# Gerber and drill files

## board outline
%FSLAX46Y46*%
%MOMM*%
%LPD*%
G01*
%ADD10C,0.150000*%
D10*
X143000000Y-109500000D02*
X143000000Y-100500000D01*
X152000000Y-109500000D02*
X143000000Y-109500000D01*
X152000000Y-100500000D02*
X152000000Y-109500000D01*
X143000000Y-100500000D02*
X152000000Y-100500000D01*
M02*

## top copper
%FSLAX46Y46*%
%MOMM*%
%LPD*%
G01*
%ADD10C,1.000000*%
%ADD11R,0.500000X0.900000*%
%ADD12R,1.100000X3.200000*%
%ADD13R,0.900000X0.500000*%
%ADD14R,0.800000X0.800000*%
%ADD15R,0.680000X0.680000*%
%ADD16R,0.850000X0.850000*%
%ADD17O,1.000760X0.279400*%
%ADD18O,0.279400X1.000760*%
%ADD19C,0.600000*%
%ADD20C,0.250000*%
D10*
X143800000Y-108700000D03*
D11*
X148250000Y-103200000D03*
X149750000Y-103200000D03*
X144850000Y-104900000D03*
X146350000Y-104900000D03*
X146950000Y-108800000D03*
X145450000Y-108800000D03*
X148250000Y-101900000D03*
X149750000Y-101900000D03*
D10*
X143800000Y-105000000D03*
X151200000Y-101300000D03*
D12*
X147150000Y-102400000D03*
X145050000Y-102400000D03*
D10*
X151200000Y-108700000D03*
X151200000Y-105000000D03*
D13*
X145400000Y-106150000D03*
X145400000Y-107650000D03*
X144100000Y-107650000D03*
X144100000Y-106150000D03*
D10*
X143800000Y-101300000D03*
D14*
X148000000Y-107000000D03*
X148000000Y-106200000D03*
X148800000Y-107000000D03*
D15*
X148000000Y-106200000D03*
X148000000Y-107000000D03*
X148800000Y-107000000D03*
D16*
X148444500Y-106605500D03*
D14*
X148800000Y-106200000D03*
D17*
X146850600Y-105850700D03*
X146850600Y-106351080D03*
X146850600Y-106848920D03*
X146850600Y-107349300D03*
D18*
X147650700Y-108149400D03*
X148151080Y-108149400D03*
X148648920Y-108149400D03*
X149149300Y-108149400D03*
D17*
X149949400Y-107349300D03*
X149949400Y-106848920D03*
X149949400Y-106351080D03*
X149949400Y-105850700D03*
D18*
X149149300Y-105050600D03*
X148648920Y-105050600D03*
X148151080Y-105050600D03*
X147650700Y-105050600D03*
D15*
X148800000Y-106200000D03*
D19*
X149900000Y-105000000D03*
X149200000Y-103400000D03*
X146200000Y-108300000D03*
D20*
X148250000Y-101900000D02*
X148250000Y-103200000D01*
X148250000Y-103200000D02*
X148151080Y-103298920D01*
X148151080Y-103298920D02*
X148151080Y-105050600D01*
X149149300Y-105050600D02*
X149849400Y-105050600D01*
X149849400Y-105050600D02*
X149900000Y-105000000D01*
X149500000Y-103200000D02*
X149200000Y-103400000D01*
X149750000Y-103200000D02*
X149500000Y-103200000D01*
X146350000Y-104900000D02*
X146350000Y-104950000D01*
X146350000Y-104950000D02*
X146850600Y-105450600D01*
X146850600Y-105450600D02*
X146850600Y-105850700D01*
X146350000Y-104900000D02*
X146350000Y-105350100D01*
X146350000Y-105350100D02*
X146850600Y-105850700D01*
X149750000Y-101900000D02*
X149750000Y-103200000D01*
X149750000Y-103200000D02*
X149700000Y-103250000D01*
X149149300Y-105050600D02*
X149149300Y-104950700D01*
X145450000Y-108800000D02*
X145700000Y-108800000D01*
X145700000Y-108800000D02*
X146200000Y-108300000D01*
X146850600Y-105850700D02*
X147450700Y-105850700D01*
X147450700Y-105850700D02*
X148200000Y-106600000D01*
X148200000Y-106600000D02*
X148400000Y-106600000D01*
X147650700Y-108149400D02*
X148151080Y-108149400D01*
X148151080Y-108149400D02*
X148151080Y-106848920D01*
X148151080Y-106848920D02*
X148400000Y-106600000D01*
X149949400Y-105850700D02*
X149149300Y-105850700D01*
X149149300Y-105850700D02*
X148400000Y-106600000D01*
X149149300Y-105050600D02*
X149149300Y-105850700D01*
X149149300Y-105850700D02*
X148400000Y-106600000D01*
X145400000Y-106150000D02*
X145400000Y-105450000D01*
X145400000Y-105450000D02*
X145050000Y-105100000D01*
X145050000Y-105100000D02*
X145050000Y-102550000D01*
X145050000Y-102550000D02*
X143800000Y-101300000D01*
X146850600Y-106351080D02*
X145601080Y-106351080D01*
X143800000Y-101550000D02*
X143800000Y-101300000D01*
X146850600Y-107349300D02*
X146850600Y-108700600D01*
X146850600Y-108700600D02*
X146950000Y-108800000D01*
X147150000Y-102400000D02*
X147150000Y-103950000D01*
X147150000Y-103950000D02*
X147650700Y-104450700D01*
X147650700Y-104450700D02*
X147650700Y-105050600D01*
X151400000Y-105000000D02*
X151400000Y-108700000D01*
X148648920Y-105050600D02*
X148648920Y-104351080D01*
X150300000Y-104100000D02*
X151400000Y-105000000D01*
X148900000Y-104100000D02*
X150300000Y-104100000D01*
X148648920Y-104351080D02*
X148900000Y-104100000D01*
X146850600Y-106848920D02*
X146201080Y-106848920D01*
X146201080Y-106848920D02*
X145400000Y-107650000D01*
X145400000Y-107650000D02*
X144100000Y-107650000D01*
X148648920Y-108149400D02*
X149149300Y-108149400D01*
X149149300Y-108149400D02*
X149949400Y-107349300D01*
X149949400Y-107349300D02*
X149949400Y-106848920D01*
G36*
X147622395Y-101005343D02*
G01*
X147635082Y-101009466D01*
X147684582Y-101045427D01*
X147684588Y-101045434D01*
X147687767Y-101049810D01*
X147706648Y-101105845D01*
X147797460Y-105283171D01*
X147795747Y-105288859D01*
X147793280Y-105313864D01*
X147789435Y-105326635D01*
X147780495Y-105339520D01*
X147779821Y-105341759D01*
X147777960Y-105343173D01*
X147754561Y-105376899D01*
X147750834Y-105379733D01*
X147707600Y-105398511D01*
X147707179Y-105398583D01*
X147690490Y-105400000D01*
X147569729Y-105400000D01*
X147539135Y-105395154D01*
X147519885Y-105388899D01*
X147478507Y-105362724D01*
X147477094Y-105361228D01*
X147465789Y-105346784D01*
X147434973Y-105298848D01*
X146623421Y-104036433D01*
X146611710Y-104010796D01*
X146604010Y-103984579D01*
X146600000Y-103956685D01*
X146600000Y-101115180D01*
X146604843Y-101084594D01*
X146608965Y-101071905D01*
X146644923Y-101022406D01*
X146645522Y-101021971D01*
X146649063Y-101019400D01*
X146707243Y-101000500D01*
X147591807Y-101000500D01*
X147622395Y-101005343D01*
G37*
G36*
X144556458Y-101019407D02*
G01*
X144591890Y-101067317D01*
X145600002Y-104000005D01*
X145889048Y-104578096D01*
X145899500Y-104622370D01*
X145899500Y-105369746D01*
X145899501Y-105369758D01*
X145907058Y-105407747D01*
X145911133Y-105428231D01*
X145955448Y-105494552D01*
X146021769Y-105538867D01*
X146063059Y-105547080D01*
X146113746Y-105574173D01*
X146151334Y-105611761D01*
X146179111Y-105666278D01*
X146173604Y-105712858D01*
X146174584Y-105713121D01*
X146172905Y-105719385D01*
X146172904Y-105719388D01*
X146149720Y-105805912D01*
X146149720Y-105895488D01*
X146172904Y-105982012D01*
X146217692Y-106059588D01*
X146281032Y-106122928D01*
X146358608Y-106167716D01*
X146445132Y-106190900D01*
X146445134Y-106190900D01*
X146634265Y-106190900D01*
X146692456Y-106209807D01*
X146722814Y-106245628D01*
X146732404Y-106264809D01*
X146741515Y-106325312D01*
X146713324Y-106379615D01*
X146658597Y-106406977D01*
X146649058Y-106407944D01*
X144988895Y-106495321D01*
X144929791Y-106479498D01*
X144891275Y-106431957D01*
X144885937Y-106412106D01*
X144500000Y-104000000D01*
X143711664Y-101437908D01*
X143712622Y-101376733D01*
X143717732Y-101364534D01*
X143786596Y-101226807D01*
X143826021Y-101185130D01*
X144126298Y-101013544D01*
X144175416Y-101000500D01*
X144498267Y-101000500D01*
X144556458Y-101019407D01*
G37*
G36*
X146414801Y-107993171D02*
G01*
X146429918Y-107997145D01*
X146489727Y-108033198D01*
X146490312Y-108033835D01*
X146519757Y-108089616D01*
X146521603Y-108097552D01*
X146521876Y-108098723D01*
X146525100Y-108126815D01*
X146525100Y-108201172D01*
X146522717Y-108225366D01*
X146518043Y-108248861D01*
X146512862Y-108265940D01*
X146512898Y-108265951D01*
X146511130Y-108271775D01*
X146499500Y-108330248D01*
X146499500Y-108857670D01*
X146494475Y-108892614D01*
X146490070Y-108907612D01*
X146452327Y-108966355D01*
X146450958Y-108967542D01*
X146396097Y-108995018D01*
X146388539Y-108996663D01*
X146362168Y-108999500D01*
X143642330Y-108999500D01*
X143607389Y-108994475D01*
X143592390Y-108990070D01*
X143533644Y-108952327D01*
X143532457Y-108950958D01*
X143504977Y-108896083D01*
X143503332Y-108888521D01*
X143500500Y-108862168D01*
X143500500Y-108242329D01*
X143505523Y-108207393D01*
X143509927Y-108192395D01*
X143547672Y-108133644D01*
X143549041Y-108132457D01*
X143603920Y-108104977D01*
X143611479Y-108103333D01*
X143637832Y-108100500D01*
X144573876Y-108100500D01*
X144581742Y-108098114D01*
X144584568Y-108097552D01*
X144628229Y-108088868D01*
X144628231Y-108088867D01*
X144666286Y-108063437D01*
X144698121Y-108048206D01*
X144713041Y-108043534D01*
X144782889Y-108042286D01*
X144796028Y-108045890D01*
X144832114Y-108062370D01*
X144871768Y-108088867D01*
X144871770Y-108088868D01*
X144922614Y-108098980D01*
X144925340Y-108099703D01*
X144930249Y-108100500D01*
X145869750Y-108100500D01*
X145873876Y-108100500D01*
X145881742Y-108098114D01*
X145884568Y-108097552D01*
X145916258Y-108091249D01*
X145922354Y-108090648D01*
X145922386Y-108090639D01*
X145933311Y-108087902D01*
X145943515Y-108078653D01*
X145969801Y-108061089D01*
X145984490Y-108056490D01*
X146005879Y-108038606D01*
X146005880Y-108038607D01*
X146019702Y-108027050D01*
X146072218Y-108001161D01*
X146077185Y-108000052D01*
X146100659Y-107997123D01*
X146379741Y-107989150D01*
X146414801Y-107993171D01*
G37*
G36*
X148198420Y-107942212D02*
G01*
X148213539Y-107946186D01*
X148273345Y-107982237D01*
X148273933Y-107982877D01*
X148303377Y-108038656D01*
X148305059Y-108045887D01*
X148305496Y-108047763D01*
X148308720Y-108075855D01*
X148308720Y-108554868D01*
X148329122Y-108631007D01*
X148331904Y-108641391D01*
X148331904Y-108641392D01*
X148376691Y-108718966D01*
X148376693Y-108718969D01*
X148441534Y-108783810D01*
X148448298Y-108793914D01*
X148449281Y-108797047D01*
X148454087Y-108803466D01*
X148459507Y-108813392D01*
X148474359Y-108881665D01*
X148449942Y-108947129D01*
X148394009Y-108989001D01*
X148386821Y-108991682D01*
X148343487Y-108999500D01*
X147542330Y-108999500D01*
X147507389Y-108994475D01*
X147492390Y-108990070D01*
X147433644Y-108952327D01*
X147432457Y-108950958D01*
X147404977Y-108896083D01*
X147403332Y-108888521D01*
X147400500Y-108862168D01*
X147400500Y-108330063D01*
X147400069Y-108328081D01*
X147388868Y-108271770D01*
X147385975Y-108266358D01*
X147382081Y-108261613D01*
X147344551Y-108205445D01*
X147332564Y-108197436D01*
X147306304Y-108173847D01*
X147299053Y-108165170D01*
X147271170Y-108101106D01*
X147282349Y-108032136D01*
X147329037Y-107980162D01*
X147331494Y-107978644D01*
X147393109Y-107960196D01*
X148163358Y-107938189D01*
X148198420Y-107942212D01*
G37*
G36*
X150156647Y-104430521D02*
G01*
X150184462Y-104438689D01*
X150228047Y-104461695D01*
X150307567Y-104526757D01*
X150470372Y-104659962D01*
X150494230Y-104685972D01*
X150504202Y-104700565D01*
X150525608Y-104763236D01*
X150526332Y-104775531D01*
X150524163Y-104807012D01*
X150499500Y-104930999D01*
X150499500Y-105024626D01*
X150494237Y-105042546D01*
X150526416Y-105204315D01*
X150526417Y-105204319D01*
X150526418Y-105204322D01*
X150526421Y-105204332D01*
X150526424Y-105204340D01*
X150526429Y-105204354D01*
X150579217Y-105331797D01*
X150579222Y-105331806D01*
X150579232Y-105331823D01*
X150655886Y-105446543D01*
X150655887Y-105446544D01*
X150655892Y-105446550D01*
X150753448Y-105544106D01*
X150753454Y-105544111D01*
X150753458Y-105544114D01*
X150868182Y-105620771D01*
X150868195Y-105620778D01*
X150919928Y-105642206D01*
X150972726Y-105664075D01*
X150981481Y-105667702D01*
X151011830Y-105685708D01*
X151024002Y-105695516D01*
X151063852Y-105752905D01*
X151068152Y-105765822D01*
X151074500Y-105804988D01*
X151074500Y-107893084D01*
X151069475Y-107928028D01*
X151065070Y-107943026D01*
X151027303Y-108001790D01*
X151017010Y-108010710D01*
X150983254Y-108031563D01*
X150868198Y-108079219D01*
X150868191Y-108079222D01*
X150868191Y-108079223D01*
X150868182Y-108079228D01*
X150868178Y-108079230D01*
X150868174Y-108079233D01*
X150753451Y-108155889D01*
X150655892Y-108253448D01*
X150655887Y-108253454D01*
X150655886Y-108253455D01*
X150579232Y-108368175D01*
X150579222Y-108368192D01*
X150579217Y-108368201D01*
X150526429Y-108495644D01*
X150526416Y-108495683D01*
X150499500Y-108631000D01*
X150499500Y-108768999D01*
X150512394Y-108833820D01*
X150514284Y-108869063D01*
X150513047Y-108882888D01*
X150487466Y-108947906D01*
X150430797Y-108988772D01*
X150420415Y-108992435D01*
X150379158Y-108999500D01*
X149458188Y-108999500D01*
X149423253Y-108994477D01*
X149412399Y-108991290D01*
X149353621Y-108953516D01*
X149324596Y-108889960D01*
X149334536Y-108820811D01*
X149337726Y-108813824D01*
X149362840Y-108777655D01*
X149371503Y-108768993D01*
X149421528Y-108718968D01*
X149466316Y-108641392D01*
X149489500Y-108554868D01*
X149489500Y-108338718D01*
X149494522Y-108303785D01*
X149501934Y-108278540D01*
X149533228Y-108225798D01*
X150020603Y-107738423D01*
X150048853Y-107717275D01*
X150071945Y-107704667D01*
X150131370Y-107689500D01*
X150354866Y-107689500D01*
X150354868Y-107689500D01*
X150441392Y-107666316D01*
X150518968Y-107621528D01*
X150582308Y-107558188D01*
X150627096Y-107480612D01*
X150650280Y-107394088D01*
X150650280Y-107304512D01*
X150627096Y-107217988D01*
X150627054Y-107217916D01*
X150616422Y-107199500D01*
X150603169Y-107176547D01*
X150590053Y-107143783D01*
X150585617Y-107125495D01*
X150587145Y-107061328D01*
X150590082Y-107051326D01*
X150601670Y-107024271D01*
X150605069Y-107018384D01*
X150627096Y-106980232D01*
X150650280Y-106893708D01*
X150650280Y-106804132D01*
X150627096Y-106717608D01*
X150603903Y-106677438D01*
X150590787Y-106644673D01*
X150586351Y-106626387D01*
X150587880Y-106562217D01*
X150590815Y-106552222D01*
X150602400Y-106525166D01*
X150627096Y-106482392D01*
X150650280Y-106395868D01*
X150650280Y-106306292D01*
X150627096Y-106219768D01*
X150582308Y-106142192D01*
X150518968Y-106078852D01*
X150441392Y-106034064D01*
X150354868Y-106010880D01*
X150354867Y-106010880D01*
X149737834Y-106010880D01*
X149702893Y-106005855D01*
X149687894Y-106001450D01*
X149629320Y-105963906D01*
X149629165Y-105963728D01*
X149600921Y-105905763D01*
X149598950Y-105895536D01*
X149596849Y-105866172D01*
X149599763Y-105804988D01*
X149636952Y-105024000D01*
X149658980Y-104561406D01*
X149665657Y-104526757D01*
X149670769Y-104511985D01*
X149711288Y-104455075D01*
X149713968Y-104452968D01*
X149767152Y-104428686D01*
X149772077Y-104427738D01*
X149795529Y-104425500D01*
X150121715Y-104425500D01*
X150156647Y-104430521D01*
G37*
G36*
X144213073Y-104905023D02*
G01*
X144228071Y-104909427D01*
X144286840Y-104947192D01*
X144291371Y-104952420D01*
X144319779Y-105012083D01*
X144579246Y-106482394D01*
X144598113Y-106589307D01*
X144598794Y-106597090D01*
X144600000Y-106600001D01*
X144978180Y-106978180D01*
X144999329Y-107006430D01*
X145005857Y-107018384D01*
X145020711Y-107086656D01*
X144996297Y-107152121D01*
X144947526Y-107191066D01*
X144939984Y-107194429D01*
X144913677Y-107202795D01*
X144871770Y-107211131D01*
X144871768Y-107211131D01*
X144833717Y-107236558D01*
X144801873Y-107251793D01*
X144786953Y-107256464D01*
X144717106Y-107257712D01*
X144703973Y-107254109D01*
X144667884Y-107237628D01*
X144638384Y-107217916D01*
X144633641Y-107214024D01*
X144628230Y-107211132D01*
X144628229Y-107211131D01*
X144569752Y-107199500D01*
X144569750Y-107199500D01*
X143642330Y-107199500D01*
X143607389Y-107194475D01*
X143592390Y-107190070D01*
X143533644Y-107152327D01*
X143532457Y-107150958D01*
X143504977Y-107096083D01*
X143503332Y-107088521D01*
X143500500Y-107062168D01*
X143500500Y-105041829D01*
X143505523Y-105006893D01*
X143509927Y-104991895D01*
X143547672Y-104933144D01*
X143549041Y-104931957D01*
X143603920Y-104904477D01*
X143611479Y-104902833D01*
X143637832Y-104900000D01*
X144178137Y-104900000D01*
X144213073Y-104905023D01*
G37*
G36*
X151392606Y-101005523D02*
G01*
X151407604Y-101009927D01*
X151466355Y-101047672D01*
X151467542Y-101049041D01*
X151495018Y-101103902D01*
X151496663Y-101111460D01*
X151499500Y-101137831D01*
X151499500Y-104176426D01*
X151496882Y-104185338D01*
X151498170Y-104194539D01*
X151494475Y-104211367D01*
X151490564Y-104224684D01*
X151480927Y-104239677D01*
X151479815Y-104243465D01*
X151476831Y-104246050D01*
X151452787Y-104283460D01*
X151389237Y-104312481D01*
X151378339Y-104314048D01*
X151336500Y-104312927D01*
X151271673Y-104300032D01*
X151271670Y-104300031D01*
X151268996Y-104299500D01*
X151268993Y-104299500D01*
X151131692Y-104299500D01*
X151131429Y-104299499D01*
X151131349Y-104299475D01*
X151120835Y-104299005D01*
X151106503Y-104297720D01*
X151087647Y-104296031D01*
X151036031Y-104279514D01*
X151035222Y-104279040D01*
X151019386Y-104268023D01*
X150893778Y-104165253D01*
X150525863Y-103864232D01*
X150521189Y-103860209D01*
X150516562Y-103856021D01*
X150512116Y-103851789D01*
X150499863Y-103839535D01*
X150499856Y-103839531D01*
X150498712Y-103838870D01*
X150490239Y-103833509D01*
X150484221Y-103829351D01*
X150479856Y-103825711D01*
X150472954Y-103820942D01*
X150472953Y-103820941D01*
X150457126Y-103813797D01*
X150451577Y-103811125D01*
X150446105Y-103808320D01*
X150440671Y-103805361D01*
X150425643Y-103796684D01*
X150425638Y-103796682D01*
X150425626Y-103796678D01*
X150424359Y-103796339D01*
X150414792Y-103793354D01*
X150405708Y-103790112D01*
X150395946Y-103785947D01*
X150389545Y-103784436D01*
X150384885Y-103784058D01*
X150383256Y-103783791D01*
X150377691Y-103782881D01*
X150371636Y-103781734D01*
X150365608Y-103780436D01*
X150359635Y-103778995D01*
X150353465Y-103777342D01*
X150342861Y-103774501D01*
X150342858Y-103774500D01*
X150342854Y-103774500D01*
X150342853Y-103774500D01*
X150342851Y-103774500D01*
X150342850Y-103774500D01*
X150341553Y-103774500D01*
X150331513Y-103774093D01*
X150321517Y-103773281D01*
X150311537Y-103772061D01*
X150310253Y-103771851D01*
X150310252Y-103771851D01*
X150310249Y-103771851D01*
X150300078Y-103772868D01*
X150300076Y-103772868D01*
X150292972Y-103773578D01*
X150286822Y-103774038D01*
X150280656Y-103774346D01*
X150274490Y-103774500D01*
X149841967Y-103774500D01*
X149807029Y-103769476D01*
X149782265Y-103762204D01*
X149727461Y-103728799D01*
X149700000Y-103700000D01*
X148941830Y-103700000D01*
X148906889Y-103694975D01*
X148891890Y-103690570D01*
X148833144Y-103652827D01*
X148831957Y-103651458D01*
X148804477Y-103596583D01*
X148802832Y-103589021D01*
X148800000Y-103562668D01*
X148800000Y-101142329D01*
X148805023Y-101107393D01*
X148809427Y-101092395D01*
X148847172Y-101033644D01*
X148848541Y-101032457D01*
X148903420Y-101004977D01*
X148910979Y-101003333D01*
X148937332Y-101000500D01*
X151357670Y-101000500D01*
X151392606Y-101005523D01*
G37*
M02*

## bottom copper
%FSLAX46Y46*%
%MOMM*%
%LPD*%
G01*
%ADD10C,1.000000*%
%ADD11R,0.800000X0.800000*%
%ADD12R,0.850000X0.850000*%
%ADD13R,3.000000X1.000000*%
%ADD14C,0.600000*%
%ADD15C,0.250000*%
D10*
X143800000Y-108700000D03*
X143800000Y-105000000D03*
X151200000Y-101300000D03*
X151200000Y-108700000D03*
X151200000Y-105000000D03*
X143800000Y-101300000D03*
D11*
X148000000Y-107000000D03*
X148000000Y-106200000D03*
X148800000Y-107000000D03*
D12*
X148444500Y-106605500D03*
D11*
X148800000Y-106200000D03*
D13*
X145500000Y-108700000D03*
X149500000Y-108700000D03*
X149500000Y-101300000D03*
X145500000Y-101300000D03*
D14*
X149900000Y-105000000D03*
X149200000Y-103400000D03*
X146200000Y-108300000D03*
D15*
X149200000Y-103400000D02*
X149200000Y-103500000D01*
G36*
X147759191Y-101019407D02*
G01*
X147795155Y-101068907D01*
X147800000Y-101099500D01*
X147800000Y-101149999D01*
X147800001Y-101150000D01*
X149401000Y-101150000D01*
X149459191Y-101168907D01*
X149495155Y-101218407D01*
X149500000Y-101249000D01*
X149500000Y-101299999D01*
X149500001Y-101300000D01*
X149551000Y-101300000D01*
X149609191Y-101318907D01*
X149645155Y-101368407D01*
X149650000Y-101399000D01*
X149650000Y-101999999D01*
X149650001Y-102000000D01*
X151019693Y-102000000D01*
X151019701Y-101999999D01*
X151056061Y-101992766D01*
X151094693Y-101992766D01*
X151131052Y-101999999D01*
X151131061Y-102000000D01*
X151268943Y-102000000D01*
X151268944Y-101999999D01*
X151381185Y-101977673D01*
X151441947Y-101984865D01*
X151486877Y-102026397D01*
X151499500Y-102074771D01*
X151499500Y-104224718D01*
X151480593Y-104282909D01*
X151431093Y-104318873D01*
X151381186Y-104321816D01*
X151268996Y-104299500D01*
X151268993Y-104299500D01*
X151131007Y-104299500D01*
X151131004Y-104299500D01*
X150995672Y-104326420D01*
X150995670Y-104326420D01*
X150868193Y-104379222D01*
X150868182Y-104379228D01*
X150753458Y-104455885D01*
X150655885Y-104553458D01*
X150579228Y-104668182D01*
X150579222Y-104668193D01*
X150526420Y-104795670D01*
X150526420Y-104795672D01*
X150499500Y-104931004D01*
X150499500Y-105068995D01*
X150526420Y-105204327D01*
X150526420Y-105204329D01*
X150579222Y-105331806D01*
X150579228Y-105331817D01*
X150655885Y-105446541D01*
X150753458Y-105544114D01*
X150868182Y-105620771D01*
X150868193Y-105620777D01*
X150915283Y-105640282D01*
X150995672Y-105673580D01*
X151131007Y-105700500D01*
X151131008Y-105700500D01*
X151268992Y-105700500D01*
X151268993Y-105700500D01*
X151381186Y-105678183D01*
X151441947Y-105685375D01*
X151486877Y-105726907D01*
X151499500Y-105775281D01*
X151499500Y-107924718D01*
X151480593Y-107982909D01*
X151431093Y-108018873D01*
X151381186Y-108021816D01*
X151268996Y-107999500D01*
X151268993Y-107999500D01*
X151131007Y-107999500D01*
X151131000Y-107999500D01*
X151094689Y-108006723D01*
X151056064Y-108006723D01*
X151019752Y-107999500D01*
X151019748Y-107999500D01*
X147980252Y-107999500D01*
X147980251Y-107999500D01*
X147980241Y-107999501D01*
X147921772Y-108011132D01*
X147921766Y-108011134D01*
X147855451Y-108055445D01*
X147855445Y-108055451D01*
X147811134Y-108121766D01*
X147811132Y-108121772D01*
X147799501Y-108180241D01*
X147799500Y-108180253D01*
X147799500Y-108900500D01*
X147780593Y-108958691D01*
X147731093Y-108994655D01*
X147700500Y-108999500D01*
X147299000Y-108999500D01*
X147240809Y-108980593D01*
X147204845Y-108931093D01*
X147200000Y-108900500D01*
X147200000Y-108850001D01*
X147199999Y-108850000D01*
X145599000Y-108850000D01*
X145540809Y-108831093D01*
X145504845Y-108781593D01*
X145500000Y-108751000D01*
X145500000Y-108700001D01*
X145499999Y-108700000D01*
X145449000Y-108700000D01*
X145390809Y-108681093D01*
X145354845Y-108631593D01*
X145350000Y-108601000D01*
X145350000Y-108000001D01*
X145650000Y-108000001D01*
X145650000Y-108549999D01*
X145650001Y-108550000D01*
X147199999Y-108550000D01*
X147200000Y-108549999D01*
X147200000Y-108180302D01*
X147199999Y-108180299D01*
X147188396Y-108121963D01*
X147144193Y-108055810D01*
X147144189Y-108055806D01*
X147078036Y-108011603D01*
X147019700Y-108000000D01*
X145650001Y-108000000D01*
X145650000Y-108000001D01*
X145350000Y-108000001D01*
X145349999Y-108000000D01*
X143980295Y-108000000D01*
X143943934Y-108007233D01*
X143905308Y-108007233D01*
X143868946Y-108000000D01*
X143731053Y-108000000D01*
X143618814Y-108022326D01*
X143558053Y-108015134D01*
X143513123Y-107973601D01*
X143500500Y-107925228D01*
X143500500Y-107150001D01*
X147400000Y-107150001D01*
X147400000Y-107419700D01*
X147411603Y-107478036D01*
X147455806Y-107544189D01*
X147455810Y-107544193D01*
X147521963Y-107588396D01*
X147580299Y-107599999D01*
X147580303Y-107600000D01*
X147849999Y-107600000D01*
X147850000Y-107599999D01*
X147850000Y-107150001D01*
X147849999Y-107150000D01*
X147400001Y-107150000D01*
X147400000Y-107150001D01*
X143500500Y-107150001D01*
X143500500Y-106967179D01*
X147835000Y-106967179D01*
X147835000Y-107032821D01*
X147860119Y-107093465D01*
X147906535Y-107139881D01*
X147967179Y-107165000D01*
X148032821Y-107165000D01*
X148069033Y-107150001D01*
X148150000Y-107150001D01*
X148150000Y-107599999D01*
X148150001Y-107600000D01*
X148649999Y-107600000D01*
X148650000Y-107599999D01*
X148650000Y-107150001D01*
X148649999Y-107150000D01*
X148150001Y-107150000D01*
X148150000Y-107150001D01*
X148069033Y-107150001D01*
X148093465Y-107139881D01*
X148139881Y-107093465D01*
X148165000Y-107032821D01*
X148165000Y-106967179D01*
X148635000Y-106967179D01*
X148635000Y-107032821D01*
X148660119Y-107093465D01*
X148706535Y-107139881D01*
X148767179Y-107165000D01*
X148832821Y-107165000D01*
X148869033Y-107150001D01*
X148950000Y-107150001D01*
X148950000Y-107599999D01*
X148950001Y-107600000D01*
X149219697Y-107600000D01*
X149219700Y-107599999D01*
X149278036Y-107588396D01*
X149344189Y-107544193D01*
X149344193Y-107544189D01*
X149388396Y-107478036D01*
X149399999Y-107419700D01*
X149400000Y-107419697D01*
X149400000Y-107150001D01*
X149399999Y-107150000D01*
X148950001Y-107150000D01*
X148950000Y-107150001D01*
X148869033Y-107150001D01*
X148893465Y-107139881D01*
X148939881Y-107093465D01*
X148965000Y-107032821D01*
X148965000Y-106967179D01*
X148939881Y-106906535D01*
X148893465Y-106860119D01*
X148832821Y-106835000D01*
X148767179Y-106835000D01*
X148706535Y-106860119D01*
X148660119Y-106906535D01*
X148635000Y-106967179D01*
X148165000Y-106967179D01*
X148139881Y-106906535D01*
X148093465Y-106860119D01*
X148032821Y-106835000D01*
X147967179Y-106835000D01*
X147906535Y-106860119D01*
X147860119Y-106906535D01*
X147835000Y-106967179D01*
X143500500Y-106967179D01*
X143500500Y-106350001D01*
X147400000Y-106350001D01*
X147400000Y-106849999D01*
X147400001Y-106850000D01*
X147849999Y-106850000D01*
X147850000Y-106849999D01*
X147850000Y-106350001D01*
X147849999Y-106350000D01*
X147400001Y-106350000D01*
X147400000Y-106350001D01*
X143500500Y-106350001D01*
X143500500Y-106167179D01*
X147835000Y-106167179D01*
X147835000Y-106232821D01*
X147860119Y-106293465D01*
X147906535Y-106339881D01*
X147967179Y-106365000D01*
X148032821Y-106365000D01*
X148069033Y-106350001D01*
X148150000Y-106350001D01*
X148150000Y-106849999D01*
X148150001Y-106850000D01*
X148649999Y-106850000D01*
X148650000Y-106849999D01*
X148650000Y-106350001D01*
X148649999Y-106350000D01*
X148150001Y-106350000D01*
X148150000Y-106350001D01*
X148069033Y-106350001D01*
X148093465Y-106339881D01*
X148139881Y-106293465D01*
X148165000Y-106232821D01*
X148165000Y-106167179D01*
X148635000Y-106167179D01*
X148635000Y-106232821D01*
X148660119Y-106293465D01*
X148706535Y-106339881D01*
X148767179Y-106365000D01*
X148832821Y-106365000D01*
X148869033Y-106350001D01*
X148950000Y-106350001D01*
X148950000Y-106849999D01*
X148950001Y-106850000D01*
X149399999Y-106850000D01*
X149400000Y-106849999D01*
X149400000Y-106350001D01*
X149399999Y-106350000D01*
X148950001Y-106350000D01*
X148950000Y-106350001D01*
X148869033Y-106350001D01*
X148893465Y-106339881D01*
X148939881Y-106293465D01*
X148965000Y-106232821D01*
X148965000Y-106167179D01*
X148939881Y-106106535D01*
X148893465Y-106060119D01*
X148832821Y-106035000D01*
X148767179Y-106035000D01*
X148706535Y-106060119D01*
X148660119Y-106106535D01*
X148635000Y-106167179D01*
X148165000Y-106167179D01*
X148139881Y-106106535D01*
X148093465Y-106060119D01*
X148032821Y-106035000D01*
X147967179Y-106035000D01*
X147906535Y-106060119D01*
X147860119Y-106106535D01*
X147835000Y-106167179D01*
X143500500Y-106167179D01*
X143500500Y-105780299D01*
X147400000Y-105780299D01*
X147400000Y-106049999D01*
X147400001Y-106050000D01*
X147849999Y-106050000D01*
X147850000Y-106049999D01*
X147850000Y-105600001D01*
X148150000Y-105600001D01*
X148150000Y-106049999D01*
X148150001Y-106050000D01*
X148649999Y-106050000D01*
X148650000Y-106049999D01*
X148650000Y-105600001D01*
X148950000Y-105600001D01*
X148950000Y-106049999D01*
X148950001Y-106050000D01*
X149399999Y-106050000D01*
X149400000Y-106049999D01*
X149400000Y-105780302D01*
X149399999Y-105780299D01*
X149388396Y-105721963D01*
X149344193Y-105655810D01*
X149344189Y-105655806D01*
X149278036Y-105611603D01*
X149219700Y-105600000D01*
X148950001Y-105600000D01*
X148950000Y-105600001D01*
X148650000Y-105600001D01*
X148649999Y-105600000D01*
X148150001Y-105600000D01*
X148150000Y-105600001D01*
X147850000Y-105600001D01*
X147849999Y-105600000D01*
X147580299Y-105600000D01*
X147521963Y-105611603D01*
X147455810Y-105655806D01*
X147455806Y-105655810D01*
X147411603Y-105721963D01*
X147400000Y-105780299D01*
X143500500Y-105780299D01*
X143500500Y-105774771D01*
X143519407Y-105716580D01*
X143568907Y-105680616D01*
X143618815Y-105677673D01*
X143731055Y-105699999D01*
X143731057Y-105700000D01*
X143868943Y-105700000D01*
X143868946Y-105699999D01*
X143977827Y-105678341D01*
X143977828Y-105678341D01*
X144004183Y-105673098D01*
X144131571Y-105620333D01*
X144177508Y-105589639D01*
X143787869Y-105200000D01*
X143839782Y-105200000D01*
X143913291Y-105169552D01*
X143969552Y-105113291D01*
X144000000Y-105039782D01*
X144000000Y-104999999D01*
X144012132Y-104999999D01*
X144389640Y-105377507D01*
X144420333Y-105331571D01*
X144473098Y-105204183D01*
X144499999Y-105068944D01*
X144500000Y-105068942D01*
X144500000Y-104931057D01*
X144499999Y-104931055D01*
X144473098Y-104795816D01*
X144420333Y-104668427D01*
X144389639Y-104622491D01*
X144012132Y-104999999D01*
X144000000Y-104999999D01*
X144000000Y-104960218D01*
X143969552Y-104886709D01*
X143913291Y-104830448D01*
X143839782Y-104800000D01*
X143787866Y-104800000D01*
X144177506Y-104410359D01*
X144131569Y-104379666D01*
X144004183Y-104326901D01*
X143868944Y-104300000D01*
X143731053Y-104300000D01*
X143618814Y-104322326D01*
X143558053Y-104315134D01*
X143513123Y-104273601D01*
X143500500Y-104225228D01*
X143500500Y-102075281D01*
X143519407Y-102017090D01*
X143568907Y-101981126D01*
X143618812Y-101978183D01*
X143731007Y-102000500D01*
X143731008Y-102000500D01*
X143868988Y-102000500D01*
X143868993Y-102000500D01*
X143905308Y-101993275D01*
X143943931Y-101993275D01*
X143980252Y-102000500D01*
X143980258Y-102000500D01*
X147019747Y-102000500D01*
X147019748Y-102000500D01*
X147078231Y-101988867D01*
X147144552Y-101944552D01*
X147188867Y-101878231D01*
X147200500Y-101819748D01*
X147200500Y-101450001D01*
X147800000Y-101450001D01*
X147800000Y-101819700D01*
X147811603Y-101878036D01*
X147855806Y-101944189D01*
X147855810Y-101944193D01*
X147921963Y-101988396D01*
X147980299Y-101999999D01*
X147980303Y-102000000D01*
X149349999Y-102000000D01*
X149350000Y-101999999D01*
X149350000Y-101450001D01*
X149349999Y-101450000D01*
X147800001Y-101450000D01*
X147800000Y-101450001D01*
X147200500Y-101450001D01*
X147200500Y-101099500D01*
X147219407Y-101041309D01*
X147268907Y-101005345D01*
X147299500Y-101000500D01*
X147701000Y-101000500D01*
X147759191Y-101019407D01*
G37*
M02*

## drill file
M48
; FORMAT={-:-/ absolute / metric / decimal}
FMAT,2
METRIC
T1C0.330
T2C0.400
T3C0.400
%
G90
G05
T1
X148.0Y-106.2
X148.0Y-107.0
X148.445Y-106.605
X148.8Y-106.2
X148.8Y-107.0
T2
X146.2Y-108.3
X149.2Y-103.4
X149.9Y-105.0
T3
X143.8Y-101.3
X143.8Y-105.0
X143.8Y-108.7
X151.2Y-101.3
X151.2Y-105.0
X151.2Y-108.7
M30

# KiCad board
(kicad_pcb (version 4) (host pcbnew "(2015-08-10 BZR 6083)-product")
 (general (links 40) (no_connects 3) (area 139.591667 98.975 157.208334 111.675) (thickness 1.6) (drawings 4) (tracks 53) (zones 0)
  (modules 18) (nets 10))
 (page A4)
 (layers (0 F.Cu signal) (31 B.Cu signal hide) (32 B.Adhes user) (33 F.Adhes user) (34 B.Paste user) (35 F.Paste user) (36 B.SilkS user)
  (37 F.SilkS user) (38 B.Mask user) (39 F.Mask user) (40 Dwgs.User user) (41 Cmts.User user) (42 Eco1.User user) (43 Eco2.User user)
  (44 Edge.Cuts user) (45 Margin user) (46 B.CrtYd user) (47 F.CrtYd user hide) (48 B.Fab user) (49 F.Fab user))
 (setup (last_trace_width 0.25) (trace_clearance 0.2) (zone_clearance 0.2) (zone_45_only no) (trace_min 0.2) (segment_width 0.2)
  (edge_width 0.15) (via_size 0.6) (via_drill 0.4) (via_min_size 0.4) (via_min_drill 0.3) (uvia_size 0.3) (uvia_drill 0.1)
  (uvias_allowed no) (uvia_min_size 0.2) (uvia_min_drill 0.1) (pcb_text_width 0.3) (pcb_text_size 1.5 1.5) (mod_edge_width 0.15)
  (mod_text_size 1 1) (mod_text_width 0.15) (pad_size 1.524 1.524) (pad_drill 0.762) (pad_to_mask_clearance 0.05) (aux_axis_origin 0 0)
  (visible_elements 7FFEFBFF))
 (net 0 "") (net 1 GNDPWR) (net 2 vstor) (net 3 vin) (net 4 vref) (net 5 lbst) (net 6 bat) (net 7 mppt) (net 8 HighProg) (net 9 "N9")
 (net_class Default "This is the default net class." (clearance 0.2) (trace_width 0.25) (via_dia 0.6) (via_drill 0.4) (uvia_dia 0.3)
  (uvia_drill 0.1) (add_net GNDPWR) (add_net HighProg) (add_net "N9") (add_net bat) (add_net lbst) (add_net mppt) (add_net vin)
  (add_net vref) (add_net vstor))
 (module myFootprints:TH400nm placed (layer F.Cu) (at 143.8 108.7)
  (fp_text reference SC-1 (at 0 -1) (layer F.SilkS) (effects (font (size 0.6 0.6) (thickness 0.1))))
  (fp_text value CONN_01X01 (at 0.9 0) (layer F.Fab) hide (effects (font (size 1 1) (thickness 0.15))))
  (pad 1 thru_hole circle (at 0 0) (size 1 1) (drill 0.4) (layers *.Cu *.Mask F.SilkS) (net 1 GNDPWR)))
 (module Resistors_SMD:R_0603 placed (layer F.Cu) (at 149 103.2)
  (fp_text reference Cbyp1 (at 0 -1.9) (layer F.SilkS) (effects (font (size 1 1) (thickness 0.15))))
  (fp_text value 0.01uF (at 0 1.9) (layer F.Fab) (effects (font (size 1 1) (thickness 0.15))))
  (pad 1 smd rect (at -0.75 0) (size 0.5 0.9) (layers F.Cu F.Paste F.Mask) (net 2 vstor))
  (pad 2 smd rect (at 0.75 0) (size 0.5 0.9) (layers F.Cu F.Paste F.Mask) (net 1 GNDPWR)))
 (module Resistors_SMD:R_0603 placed (layer F.Cu) (at 145.6 104.9)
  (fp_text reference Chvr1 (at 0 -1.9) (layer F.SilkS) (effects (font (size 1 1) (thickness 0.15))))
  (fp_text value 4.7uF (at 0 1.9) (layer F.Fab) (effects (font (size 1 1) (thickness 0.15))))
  (pad 1 smd rect (at -0.75 0) (size 0.5 0.9) (layers F.Cu F.Paste F.Mask) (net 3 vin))
  (pad 2 smd rect (at 0.75 0) (size 0.5 0.9) (layers F.Cu F.Paste F.Mask) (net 1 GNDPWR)))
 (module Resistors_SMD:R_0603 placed (layer F.Cu) (at 146.2 108.8 180)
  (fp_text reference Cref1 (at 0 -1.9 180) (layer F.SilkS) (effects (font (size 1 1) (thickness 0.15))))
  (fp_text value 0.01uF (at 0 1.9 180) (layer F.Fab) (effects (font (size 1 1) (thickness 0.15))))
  (pad 1 smd rect (at -0.75 0 180) (size 0.5 0.9) (layers F.Cu F.Paste F.Mask) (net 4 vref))
  (pad 2 smd rect (at 0.75 0 180) (size 0.5 0.9) (layers F.Cu F.Paste F.Mask) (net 1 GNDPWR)))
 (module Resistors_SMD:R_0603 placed (layer F.Cu) (at 149 101.9)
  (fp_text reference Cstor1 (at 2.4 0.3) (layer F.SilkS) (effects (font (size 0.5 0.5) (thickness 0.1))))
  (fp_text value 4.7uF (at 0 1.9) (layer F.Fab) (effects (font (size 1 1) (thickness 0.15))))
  (pad 1 smd rect (at -0.75 0) (size 0.5 0.9) (layers F.Cu F.Paste F.Mask) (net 2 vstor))
  (pad 2 smd rect (at 0.75 0) (size 0.5 0.9) (layers F.Cu F.Paste F.Mask) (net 1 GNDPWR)))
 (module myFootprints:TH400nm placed (layer F.Cu) (at 143.8 105)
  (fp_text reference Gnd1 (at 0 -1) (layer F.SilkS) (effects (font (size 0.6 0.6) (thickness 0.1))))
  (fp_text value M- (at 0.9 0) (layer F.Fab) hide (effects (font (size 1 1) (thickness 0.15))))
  (pad 1 thru_hole circle (at 0 0) (size 1 1) (drill 0.4) (layers *.Cu *.Mask F.SilkS) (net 1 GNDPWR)))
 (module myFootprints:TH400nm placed (layer F.Cu) (at 151.2 101.3)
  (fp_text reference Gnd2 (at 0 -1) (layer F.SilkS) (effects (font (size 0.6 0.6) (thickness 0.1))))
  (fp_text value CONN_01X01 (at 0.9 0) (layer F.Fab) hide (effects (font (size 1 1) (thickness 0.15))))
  (pad 1 thru_hole circle (at 0 0) (size 1 1) (drill 0.4) (layers *.Cu *.Mask F.SilkS) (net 1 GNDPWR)))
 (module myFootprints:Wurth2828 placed (layer F.Cu) (at 146.1 102.4)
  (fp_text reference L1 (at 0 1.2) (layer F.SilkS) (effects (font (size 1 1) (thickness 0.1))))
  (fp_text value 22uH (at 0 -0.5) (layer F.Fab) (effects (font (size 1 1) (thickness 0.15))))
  (pad 1 smd rect (at 1.05 0) (size 1.1 3.2) (layers F.Cu F.Paste F.Mask) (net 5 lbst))
  (pad 2 smd rect (at -1.05 0) (size 1.1 3.2) (layers F.Cu F.Paste F.Mask) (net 3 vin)))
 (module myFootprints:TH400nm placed (layer F.Cu) (at 151.2 108.7)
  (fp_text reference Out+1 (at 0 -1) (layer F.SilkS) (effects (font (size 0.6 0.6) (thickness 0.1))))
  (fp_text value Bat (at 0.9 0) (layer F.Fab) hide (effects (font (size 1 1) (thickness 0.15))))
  (pad 1 thru_hole circle (at 0 0) (size 1 1) (drill 0.4) (layers *.Cu *.Mask F.SilkS) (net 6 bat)))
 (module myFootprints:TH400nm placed (layer F.Cu) (at 151.2 105)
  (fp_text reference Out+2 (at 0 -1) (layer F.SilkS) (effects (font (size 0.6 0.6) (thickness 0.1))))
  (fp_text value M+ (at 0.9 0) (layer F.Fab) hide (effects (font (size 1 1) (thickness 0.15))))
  (pad 1 thru_hole circle (at 0 0) (size 1 1) (drill 0.4) (layers *.Cu *.Mask F.SilkS) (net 6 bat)))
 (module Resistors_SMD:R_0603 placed (layer F.Cu) (at 145.4 106.9 270)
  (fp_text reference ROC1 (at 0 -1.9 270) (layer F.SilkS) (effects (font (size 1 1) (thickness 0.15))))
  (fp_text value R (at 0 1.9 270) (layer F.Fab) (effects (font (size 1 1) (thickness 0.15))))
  (pad 1 smd rect (at -0.75 0 270) (size 0.5 0.9) (layers F.Cu F.Paste F.Mask) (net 3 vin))
  (pad 2 smd rect (at 0.75 0 270) (size 0.5 0.9) (layers F.Cu F.Paste F.Mask) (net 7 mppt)))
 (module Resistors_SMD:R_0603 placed (layer F.Cu) (at 144.1 106.9 90)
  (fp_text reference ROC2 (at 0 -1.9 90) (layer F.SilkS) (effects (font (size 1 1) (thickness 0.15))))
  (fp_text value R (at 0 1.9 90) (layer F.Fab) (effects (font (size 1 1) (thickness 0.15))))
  (pad 1 smd rect (at -0.75 0 90) (size 0.5 0.9) (layers F.Cu F.Paste F.Mask) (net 7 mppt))
  (pad 2 smd rect (at 0.75 0 90) (size 0.5 0.9) (layers F.Cu F.Paste F.Mask) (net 1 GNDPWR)))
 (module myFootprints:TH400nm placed (layer F.Cu) (at 143.8 101.3)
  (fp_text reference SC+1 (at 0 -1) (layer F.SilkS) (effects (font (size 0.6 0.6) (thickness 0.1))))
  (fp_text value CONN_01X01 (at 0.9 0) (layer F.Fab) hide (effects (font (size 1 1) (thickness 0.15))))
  (pad 1 thru_hole circle (at 0 0) (size 1 1) (drill 0.4) (layers *.Cu *.Mask F.SilkS) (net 3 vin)))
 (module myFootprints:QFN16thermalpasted (layer F.Cu) (at 148.4 106.6)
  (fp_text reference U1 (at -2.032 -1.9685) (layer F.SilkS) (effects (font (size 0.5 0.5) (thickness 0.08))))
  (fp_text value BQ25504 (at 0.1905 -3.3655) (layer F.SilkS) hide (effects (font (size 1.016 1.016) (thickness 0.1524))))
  (pad 17 thru_hole rect (at -0.4 0.4) (size 0.8 0.8) (drill 0.33) (layers *.Cu *.Mask F.SilkS) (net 1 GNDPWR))
  (pad 17 thru_hole rect (at -0.4 -0.4) (size 0.8 0.8) (drill 0.33) (layers *.Cu *.Mask F.SilkS) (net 1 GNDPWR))
  (pad 17 thru_hole rect (at 0.4 0.4) (size 0.8 0.8) (drill 0.33) (layers *.Cu *.Mask F.SilkS) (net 1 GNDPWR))
  (pad 17 smd rect (at -0.4 -0.4) (size 0.68 0.68) (layers F.Cu F.Paste F.Mask) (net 1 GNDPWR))
  (pad 17 smd rect (at -0.4 0.4) (size 0.68 0.68) (layers F.Cu F.Paste F.Mask) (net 1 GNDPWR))
  (pad 17 smd rect (at 0.4 0.4) (size 0.68 0.68) (layers F.Cu F.Paste F.Mask) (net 1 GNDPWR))
  (pad 17 thru_hole rect (at 0.0445 0.0055) (size 0.85 0.85) (drill 0.33) (layers *.Cu *.Mask F.SilkS) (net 1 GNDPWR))
  (pad 17 thru_hole rect (at 0.4 -0.4) (size 0.8 0.8) (drill 0.33) (layers *.Cu *.Mask F.SilkS) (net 1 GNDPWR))
  (pad 1 smd oval (at -1.5494 -0.7493) (size 1.00076 0.2794) (layers F.Cu F.Paste F.Mask) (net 1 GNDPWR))
  (pad 2 smd oval (at -1.5494 -0.24892) (size 1.00076 0.2794) (layers F.Cu F.Paste F.Mask) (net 3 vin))
  (pad 3 smd oval (at -1.5494 0.24892) (size 1.00076 0.2794) (layers F.Cu F.Paste F.Mask) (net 7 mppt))
  (pad 4 smd oval (at -1.5494 0.7493) (size 1.00076 0.2794) (layers F.Cu F.Paste F.Mask) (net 4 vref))
  (pad 5 smd oval (at -0.7493 1.5494 90) (size 1.00076 0.2794) (layers F.Cu F.Paste F.Mask) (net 1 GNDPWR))
  (pad 6 smd oval (at -0.24892 1.5494 90) (size 1.00076 0.2794) (layers F.Cu F.Paste F.Mask) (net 1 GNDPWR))
  (pad 7 smd oval (at 0.24892 1.5494 90) (size 1.00076 0.2794) (layers F.Cu F.Paste F.Mask) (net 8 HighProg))
  (pad 8 smd oval (at 0.7493 1.5494 90) (size 1.00076 0.2794) (layers F.Cu F.Paste F.Mask) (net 8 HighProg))
  (pad 9 smd oval (at 1.5494 0.7493) (size 1.00076 0.2794) (layers F.Cu F.Paste F.Mask) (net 8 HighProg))
  (pad 10 smd oval (at 1.5494 0.24892) (size 1.00076 0.2794) (layers F.Cu F.Paste F.Mask) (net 8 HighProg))
  (pad 11 smd oval (at 1.5494 -0.24892) (size 1.00076 0.2794) (layers F.Cu F.Paste F.Mask) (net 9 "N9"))
  (pad 12 smd oval (at 1.5494 -0.7493) (size 1.00076 0.2794) (layers F.Cu F.Paste F.Mask) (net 1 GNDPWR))
  (pad 13 smd oval (at 0.7493 -1.5494 90) (size 1.00076 0.2794) (layers F.Cu F.Paste F.Mask) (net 1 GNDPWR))
  (pad 14 smd oval (at 0.24892 -1.5494 90) (size 1.00076 0.2794) (layers F.Cu F.Paste F.Mask) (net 6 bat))
  (pad 15 smd oval (at -0.24892 -1.5494 90) (size 1.00076 0.2794) (layers F.Cu F.Paste F.Mask) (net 2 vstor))
  (pad 16 smd oval (at -0.7493 -1.5494 90) (size 1.00076 0.2794) (layers F.Cu F.Paste F.Mask) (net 5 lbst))
  (pad 17 smd rect (at 0.4 -0.4) (size 0.68 0.68) (layers F.Cu F.Paste F.Mask) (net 1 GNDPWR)))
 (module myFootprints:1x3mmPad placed (layer B.Cu) (at 145.5 108.7)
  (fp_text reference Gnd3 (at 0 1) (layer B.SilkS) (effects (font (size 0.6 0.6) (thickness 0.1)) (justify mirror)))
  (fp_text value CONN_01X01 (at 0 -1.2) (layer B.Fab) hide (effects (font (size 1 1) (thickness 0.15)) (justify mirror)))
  (pad 1 smd rect (at 0 0) (size 3 1) (layers B.Cu B.Paste B.Mask) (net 1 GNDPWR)))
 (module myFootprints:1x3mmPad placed (layer B.Cu) (at 149.5 108.7)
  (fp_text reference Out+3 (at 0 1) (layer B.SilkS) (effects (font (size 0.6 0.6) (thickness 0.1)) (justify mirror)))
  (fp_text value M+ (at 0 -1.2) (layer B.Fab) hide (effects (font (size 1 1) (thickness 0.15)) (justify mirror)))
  (pad 1 smd rect (at 0 0) (size 3 1) (layers B.Cu B.Paste B.Mask) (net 6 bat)))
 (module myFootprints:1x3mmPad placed (layer B.Cu) (at 149.5 101.3)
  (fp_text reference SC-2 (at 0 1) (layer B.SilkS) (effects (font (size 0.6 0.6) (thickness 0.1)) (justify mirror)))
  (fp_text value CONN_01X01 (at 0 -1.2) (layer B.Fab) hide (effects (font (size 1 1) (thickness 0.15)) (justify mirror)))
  (pad 1 smd rect (at 0 0) (size 3 1) (layers B.Cu B.Paste B.Mask) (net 1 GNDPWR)))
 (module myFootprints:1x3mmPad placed (layer B.Cu) (at 145.5 101.3)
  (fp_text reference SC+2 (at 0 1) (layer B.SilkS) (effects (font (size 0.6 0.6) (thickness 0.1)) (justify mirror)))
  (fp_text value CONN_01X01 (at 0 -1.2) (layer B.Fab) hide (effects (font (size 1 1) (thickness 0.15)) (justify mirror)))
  (pad 1 smd rect (at 0 0) (size 3 1) (layers B.Cu B.Paste B.Mask) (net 3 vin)))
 (gr_line (start 143 109.5) (end 143 100.5) (angle 90) (layer Edge.Cuts) (width 0.15))
 (gr_line (start 152 109.5) (end 143 109.5) (angle 90) (layer Edge.Cuts) (width 0.15))
 (gr_line (start 152 100.5) (end 152 109.5) (angle 90) (layer Edge.Cuts) (width 0.15))
 (gr_line (start 143 100.5) (end 152 100.5) (angle 90) (layer Edge.Cuts) (width 0.15))
 (segment (start 148.25 101.9) (end 148.25 103.2) (width 0.25) (layer F.Cu) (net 2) (status 20))
 (segment (start 148.25 103.2) (end 148.15108 103.29892) (width 0.25) (layer F.Cu) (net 2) (status 30))
 (segment (start 148.15108 103.29892) (end 148.15108 105.0506) (width 0.25) (layer F.Cu) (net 2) (status 10))
 (segment (start 149.1493 105.0506) (end 149.8494 105.0506) (width 0.25) (layer F.Cu) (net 1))
 (via (at 149.9 105) (size 0.6) (drill 0.4) (layers F.Cu B.Cu) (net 1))
 (segment (start 149.8494 105.0506) (end 149.9 105) (width 0.25) (layer F.Cu) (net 1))
 (segment (start 149.2 103.4) (end 149.2 103.5) (width 0.25) (layer B.Cu) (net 1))
 (via (at 149.2 103.4) (size 0.6) (drill 0.4) (layers F.Cu B.Cu) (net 1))
 (segment (start 149.5 103.2) (end 149.2 103.4) (width 0.25) (layer F.Cu) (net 1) (status 10))
 (segment (start 149.75 103.2) (end 149.5 103.2) (width 0.25) (layer F.Cu) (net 1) (status 30))
 (segment (start 146.35 104.9) (end 146.35 104.95) (width 0.25) (layer F.Cu) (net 1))
 (segment (start 146.35 104.95) (end 146.8506 105.4506) (width 0.25) (layer F.Cu) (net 1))
 (segment (start 146.8506 105.4506) (end 146.8506 105.8507) (width 0.25) (layer F.Cu) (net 1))
 (segment (start 146.35 104.9) (end 146.35 105.3501) (width 0.25) (layer F.Cu) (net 1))
 (segment (start 146.35 105.3501) (end 146.8506 105.8507) (width 0.25) (layer F.Cu) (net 1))
 (segment (start 149.75 101.9) (end 149.75 103.2) (width 0.25) (layer F.Cu) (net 1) (status 20))
 (segment (start 149.75 103.2) (end 149.7 103.25) (width 0.25) (layer F.Cu) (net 1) (status 30))
 (segment (start 149.1493 105.0506) (end 149.1493 104.9507) (width 0.25) (layer F.Cu) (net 1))
 (segment (start 145.45 108.8) (end 145.7 108.8) (width 0.25) (layer F.Cu) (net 1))
 (segment (start 145.7 108.8) (end 146.2 108.3) (width 0.25) (layer F.Cu) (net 1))
 (via (at 146.2 108.3) (size 0.6) (drill 0.4) (layers F.Cu B.Cu) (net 1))
 (segment (start 146.8506 105.8507) (end 147.4507 105.8507) (width 0.25) (layer F.Cu) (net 1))
 (segment (start 147.4507 105.8507) (end 148.2 106.6) (width 0.25) (layer F.Cu) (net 1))
 (segment (start 148.2 106.6) (end 148.4 106.6) (width 0.25) (layer F.Cu) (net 1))
 (segment (start 147.6507 108.1494) (end 148.15108 108.1494) (width 0.25) (layer F.Cu) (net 1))
 (segment (start 148.15108 108.1494) (end 148.15108 106.84892) (width 0.25) (layer F.Cu) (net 1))
 (segment (start 148.15108 106.84892) (end 148.4 106.6) (width 0.25) (layer F.Cu) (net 1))
 (segment (start 149.9494 105.8507) (end 149.1493 105.8507) (width 0.25) (layer F.Cu) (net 1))
 (segment (start 149.1493 105.8507) (end 148.4 106.6) (width 0.25) (layer F.Cu) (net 1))
 (segment (start 149.1493 105.0506) (end 149.1493 105.8507) (width 0.25) (layer F.Cu) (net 1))
 (segment (start 149.1493 105.8507) (end 148.4 106.6) (width 0.25) (layer F.Cu) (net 1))
 (segment (start 145.4 106.15) (end 145.4 105.45) (width 0.25) (layer F.Cu) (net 3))
 (segment (start 145.4 105.45) (end 145.05 105.1) (width 0.25) (layer F.Cu) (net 3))
 (segment (start 145.05 105.1) (end 145.05 102.55) (width 0.25) (layer F.Cu) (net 3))
 (segment (start 145.05 102.55) (end 143.8 101.3) (width 0.25) (layer F.Cu) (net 3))
 (segment (start 146.8506 106.35108) (end 145.60108 106.35108) (width 0.25) (layer F.Cu) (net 3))
 (segment (start 143.8 101.55) (end 143.8 101.3) (width 0.25) (layer F.Cu) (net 3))
 (segment (start 146.8506 107.3493) (end 146.8506 108.7006) (width 0.25) (layer F.Cu) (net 4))
 (segment (start 146.8506 108.7006) (end 146.95 108.8) (width 0.25) (layer F.Cu) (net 4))
 (segment (start 147.15 102.4) (end 147.15 103.95) (width 0.25) (layer F.Cu) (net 5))
 (segment (start 147.15 103.95) (end 147.6507 104.4507) (width 0.25) (layer F.Cu) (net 5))
 (segment (start 147.6507 104.4507) (end 147.6507 105.0506) (width 0.25) (layer F.Cu) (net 5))
 (segment (start 151.4 105) (end 151.4 108.7) (width 0.25) (layer F.Cu) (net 6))
 (segment (start 148.64892 105.0506) (end 148.64892 104.35108) (width 0.25) (layer F.Cu) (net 6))
 (segment (start 150.3 104.1) (end 151.4 105) (width 0.25) (layer F.Cu) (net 6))
 (segment (start 148.9 104.1) (end 150.3 104.1) (width 0.25) (layer F.Cu) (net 6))
 (segment (start 148.64892 104.35108) (end 148.9 104.1) (width 0.25) (layer F.Cu) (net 6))
 (segment (start 146.8506 106.84892) (end 146.20108 106.84892) (width 0.25) (layer F.Cu) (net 7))
 (segment (start 146.20108 106.84892) (end 145.4 107.65) (width 0.25) (layer F.Cu) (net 7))
 (segment (start 145.4 107.65) (end 144.1 107.65) (width 0.25) (layer F.Cu) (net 7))
 (segment (start 148.64892 108.1494) (end 149.1493 108.1494) (width 0.25) (layer F.Cu) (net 8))
 (segment (start 149.1493 108.1494) (end 149.9494 107.3493) (width 0.25) (layer F.Cu) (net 8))
 (segment (start 149.9494 107.3493) (end 149.9494 106.84892) (width 0.25) (layer F.Cu) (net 8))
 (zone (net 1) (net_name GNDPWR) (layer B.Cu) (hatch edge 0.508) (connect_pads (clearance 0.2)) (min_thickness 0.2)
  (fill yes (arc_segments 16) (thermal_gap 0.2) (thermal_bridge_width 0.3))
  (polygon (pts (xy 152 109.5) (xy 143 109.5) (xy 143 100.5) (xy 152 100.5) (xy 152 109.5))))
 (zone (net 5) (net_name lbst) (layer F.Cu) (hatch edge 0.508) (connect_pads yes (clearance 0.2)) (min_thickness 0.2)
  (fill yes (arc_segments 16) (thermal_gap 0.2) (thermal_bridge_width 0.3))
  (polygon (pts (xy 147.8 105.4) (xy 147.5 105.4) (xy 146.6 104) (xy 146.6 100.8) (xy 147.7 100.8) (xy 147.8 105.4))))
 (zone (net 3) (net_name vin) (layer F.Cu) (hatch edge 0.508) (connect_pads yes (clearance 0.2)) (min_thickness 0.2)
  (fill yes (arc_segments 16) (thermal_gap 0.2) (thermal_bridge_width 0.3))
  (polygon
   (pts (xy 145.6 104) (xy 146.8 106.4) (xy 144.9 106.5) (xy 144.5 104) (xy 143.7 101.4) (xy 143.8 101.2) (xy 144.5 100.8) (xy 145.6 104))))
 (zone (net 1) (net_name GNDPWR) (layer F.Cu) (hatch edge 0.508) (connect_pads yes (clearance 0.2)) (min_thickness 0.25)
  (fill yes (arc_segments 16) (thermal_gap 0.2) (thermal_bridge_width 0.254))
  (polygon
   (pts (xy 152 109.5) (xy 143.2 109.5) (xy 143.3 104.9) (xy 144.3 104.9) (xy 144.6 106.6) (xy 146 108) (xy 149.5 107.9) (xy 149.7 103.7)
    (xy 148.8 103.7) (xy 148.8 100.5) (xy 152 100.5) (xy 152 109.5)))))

